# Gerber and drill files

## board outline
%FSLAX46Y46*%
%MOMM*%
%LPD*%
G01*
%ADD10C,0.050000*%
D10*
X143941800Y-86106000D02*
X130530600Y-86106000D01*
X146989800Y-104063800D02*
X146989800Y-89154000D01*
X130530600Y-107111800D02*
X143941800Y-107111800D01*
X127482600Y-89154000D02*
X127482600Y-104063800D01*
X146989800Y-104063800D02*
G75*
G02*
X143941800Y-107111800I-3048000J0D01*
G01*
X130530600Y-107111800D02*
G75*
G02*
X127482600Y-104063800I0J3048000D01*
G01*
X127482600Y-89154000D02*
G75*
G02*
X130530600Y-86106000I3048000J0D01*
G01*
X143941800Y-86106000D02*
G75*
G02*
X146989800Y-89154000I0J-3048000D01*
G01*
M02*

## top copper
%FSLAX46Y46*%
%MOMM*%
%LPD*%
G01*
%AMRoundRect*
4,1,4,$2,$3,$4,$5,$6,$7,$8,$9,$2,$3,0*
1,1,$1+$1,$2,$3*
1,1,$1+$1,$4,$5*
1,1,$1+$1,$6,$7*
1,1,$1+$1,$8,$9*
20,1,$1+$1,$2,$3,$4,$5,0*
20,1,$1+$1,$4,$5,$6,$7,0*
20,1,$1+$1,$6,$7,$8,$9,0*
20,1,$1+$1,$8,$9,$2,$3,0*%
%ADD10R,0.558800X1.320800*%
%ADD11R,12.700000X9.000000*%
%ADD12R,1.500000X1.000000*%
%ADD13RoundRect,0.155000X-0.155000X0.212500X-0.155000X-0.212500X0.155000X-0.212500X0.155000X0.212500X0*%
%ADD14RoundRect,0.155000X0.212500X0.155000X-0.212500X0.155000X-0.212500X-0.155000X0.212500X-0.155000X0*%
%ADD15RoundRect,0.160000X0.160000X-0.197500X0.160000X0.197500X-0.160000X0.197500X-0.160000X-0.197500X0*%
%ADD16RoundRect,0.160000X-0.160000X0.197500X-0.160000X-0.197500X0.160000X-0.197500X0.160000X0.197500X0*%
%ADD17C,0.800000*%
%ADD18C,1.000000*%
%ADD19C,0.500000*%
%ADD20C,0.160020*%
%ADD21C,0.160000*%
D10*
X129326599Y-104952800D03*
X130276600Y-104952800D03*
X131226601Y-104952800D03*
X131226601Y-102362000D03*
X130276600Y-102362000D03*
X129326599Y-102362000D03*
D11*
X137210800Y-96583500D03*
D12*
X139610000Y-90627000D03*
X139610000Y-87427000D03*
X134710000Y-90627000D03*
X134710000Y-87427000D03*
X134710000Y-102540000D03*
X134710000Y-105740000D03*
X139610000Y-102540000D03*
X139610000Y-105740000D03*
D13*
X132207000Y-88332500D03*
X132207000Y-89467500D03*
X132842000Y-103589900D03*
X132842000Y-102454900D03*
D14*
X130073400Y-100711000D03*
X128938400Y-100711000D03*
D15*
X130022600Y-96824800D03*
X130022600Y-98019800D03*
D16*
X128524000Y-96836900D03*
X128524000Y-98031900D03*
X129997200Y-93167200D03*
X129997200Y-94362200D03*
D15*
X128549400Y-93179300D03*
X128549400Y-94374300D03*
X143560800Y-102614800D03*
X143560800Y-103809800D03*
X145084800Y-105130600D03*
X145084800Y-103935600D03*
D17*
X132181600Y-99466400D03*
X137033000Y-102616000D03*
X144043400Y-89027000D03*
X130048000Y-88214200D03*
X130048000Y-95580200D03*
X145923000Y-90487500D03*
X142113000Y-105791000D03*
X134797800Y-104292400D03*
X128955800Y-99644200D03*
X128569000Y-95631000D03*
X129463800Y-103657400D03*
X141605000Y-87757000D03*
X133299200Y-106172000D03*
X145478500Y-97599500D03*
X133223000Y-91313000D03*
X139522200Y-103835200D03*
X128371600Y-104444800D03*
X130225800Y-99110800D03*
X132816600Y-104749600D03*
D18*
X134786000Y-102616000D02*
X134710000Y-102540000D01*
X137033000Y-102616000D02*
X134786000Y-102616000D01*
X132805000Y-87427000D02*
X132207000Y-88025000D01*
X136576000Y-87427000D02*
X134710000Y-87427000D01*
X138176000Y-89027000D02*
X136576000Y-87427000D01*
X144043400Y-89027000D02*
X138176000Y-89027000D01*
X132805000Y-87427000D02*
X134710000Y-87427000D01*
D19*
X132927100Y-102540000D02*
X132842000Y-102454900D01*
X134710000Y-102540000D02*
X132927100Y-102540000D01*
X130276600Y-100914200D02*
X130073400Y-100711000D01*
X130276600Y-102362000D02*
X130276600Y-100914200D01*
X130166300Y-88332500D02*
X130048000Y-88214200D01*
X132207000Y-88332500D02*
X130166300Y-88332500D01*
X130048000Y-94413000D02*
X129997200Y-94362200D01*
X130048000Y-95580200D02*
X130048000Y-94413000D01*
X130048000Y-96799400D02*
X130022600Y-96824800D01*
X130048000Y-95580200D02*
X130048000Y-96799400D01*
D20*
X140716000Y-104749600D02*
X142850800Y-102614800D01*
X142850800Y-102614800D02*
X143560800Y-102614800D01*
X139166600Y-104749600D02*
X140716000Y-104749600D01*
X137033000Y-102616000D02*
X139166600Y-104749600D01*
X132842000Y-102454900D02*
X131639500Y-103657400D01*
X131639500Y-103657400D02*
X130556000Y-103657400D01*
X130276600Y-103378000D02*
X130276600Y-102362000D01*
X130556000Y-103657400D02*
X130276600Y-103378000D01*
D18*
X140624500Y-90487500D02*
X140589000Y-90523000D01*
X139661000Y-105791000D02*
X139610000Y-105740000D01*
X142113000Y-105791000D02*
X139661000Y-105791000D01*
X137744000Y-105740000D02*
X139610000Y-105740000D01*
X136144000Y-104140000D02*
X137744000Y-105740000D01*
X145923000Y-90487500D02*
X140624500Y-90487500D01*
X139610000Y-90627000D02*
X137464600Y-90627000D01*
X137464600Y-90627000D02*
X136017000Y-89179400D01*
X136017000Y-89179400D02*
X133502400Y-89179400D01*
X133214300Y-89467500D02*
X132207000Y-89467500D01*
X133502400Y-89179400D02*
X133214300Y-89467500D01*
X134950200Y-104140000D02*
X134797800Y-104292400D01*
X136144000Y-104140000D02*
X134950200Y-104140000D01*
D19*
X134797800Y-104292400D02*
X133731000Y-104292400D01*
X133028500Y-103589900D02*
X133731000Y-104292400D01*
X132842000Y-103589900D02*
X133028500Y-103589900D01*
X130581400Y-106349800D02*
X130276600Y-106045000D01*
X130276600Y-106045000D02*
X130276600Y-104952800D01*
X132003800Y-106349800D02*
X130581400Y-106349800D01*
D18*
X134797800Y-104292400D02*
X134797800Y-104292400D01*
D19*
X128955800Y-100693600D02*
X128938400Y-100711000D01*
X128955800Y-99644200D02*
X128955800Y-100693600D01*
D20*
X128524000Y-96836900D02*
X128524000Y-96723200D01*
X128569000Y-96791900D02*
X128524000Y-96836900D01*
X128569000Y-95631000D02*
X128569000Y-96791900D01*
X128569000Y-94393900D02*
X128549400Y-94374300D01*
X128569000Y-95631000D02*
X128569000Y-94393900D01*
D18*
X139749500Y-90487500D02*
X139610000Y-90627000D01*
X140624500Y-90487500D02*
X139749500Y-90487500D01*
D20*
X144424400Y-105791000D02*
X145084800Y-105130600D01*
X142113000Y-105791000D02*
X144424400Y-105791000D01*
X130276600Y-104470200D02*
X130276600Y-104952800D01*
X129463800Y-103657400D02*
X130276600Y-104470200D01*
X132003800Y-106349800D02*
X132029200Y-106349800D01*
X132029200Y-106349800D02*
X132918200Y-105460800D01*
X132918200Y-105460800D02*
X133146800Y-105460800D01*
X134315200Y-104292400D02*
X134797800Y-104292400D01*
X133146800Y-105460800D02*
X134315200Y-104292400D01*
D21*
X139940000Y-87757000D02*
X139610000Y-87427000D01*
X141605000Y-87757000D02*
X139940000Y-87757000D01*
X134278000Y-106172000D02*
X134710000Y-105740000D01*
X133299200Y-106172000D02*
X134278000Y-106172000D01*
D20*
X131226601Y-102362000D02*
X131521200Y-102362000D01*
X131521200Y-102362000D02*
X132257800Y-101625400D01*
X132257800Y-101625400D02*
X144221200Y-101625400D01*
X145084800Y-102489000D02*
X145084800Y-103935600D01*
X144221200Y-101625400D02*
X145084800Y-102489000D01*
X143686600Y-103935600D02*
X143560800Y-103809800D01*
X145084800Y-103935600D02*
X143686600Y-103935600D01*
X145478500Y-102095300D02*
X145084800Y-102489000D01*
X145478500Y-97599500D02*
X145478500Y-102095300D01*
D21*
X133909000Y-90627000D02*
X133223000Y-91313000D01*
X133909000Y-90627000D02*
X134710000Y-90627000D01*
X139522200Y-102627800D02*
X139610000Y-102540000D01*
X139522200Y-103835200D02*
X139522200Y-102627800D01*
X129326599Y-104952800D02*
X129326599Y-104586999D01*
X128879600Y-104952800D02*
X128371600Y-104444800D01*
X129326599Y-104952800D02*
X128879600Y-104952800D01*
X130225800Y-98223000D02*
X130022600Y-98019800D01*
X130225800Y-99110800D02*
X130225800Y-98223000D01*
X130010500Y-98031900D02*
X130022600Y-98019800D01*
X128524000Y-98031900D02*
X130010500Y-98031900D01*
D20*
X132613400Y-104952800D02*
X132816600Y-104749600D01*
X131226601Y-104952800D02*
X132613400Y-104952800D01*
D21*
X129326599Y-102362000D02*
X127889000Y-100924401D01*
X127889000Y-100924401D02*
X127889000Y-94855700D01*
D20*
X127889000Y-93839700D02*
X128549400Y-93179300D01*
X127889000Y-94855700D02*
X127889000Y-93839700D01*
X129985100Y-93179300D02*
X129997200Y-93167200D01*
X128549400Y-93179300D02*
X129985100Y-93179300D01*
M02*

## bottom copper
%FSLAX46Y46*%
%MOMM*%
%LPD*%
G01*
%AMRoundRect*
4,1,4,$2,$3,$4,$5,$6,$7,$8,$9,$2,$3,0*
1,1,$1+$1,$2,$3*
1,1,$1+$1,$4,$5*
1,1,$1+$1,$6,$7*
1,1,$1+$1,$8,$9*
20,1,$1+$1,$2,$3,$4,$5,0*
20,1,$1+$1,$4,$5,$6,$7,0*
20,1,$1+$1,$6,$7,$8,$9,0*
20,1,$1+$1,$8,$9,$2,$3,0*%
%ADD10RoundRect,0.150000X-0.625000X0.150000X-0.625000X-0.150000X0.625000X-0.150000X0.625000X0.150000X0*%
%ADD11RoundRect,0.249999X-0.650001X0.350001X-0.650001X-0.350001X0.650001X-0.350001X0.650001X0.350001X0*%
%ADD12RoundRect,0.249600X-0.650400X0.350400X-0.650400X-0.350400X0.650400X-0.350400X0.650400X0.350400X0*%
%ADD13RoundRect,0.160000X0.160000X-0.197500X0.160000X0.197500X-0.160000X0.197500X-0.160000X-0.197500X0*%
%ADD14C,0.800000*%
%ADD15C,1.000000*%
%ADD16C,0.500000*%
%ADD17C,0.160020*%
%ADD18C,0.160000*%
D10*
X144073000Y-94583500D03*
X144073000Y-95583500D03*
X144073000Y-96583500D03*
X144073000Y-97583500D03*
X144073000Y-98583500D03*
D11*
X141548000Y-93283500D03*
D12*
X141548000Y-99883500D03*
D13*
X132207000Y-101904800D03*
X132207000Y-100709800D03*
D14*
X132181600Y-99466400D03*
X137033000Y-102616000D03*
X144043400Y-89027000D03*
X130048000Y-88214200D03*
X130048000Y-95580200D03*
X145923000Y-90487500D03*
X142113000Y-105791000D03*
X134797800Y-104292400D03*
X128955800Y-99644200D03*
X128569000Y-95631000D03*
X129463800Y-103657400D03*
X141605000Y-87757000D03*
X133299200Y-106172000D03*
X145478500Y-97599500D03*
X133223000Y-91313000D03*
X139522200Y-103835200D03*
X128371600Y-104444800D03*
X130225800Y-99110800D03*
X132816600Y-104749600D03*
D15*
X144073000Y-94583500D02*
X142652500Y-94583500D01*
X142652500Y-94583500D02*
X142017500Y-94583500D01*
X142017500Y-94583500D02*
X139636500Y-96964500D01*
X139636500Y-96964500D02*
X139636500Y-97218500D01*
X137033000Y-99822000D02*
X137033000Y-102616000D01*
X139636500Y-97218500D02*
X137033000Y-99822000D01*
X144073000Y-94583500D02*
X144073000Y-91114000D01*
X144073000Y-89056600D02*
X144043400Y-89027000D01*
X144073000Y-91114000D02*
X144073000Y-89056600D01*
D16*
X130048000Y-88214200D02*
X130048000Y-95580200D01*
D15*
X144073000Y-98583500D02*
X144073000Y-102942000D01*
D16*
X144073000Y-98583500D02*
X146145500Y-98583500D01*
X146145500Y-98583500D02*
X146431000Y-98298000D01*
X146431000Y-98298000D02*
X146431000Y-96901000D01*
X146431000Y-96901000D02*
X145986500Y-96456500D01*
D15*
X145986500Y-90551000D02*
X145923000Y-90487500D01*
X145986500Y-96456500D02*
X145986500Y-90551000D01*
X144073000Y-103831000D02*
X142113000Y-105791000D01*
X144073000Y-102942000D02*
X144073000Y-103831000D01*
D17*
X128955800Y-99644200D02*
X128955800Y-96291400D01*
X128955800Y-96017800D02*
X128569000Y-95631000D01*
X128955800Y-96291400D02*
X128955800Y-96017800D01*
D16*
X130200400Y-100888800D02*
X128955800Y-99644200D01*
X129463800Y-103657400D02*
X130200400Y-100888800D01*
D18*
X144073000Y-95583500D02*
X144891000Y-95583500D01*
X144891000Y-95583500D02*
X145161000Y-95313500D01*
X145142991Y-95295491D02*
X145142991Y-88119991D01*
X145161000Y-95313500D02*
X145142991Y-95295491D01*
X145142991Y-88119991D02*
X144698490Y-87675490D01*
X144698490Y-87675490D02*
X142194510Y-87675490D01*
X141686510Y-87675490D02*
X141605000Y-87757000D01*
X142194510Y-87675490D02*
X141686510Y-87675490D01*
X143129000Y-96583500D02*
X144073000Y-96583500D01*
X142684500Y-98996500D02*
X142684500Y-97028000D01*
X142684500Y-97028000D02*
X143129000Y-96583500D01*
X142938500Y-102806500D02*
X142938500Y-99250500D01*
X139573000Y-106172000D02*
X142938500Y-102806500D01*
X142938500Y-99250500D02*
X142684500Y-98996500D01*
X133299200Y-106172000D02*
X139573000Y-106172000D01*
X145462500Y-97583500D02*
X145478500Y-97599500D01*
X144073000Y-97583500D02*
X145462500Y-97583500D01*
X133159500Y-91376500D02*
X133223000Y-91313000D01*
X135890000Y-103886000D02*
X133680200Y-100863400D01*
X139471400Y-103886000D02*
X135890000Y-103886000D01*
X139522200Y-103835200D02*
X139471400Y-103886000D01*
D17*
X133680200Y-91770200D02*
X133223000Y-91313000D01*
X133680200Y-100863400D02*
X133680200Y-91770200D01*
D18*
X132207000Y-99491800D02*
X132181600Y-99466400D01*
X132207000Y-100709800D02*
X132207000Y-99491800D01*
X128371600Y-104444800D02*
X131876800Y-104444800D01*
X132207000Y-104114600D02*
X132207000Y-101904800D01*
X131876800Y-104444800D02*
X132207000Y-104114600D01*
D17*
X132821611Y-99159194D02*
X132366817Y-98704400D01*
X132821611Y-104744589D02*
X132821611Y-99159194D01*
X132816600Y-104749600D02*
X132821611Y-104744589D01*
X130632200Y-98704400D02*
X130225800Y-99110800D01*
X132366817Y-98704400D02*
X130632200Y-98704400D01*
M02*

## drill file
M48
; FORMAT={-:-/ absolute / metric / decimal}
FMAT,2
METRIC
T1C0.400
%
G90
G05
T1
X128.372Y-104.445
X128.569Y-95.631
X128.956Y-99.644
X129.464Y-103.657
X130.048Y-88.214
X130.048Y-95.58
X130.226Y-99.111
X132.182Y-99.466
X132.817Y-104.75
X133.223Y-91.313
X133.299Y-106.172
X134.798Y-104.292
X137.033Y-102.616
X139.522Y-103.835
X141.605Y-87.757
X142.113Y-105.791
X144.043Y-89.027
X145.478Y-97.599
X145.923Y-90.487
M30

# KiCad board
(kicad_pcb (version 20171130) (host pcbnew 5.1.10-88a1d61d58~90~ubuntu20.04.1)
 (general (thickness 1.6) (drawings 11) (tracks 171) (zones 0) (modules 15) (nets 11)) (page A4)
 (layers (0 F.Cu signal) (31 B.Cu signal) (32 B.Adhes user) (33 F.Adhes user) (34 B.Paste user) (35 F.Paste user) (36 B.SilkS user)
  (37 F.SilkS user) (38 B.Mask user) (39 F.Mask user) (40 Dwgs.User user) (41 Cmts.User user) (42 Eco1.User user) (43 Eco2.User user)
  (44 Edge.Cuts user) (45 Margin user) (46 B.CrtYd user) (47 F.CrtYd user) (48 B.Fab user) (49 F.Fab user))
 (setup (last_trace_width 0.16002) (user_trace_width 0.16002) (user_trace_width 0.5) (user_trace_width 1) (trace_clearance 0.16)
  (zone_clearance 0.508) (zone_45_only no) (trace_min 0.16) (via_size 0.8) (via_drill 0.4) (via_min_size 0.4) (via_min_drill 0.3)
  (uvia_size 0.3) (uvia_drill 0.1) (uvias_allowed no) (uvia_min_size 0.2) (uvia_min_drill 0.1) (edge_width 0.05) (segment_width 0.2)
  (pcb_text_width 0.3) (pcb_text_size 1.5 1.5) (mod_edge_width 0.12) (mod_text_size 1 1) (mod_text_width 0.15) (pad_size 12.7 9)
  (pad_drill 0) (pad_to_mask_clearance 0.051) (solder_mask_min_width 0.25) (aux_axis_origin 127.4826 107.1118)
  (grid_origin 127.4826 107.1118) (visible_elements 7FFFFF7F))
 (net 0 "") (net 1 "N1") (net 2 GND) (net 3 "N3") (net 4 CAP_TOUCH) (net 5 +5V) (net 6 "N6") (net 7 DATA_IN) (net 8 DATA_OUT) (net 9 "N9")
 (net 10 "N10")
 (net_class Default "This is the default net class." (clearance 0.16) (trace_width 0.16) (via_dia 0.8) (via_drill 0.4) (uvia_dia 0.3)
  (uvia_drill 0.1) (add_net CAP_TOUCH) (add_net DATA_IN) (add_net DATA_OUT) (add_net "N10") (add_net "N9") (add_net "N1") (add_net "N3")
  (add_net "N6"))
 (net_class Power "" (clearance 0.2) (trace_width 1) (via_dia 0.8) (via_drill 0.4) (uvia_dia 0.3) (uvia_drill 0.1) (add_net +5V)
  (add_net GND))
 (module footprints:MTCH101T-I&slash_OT (layer F.Cu) (at 130.2766 103.6574 90)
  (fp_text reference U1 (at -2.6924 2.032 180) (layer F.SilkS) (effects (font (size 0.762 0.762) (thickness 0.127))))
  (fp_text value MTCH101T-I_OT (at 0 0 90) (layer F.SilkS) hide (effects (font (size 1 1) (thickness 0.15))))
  (pad 1 smd rect (at -1.2954 -0.950001 90) (size 1.3208 0.5588) (layers F.Cu F.Paste F.Mask) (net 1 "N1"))
  (pad 2 smd rect (at -1.2954 0 90) (size 1.3208 0.5588) (layers F.Cu F.Paste F.Mask) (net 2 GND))
  (pad 3 smd rect (at -1.2954 0.950001 90) (size 1.3208 0.5588) (layers F.Cu F.Paste F.Mask) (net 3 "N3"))
  (pad 4 smd rect (at 1.2954 0.950001 90) (size 1.3208 0.5588) (layers F.Cu F.Paste F.Mask) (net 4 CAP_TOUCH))
  (pad 5 smd rect (at 1.2954 0 90) (size 1.3208 0.5588) (layers F.Cu F.Paste F.Mask) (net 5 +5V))
  (pad 6 smd rect (at 1.2954 -0.950001 90) (size 1.3208 0.5588) (layers F.Cu F.Paste F.Mask) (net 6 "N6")))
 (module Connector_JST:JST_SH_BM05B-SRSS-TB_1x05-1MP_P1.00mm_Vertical (layer B.Cu) (at 142.748 96.5835 270)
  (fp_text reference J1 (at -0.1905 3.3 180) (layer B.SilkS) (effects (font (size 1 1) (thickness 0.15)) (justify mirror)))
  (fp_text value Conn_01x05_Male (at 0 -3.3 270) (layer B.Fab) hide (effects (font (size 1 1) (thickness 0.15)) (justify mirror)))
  (pad 1 smd roundrect (at -2 -1.325 270) (size 0.6 1.55) (layers B.Cu B.Mask) (roundrect_rratio 0.25) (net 5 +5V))
  (pad 2 smd roundrect (at -1 -1.325 270) (size 0.6 1.55) (layers B.Cu B.Mask) (roundrect_rratio 0.25) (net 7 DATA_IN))
  (pad 3 smd roundrect (at 0 -1.325 270) (size 0.6 1.55) (layers B.Cu B.Mask) (roundrect_rratio 0.25) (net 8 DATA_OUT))
  (pad 4 smd roundrect (at 1 -1.325 270) (size 0.6 1.55) (layers B.Cu B.Mask) (roundrect_rratio 0.25) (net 4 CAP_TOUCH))
  (pad 5 smd roundrect (at 2 -1.325 270) (size 0.6 1.55) (layers B.Cu B.Mask) (roundrect_rratio 0.25) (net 2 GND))
  (pad MP smd roundrect (at -3.3 1.2 270) (size 1.2 1.8) (layers B.Cu B.Paste B.Mask) (roundrect_rratio 0.2083325))
  (pad MP smd roundrect (at 3.3 1.2 270) (size 1.2 1.8) (layers B.Cu B.Mask) (roundrect_rratio 0.208)))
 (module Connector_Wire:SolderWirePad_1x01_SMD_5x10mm (layer F.Cu) (at 136.0805 96.647)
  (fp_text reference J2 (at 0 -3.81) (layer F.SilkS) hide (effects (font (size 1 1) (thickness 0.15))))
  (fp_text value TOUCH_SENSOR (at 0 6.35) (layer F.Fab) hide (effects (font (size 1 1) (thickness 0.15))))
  (pad 1 smd rect (at 1.1303 -0.0635) (size 12.7 9) (layers F.Cu F.Mask) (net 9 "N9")))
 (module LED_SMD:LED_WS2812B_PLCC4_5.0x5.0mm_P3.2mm (layer F.Cu) (at 137.16 89.027)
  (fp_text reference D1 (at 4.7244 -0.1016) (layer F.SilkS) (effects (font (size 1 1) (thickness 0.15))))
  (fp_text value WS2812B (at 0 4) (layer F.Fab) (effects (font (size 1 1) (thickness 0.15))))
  (pad 3 smd rect (at 2.45 1.6) (size 1.5 1) (layers F.Cu F.Paste F.Mask) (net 2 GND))
  (pad 4 smd rect (at 2.45 -1.6) (size 1.5 1) (layers F.Cu F.Paste F.Mask) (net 7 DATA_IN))
  (pad 2 smd rect (at -2.45 1.6) (size 1.5 1) (layers F.Cu F.Paste F.Mask) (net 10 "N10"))
  (pad 1 smd rect (at -2.45 -1.6) (size 1.5 1) (layers F.Cu F.Paste F.Mask) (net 5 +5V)))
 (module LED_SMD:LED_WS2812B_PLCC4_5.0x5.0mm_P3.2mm (layer F.Cu) (at 137.16 104.14)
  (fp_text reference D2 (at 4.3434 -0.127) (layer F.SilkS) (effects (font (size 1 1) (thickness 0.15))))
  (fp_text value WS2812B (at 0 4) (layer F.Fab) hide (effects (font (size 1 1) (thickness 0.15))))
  (pad 1 smd rect (at -2.45 -1.6) (size 1.5 1) (layers F.Cu F.Paste F.Mask) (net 5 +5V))
  (pad 2 smd rect (at -2.45 1.6) (size 1.5 1) (layers F.Cu F.Paste F.Mask) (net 8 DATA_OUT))
  (pad 4 smd rect (at 2.45 -1.6) (size 1.5 1) (layers F.Cu F.Paste F.Mask) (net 10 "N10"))
  (pad 3 smd rect (at 2.45 1.6) (size 1.5 1) (layers F.Cu F.Paste F.Mask) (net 2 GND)))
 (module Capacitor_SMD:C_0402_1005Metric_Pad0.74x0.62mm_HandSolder (layer F.Cu) (at 132.207 88.9 270)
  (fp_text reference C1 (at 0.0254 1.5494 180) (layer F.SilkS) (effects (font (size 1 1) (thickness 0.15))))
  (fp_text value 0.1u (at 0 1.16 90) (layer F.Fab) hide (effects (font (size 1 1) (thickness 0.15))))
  (pad 1 smd roundrect (at -0.5675 0 270) (size 0.735 0.62) (layers F.Cu F.Paste F.Mask) (roundrect_rratio 0.25) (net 5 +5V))
  (pad 2 smd roundrect (at 0.5675 0 270) (size 0.735 0.62) (layers F.Cu F.Paste F.Mask) (roundrect_rratio 0.25) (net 2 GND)))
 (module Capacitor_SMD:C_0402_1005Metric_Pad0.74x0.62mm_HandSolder (layer F.Cu) (at 132.842 103.0224 270)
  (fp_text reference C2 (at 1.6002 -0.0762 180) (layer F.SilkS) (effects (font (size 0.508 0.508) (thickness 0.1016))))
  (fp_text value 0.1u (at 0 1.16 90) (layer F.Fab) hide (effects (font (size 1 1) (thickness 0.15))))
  (pad 2 smd roundrect (at 0.5675 0 270) (size 0.735 0.62) (layers F.Cu F.Paste F.Mask) (roundrect_rratio 0.25) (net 2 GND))
  (pad 1 smd roundrect (at -0.5675 0 270) (size 0.735 0.62) (layers F.Cu F.Paste F.Mask) (roundrect_rratio 0.25) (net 5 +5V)))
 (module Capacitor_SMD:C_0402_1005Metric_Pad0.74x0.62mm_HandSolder (layer F.Cu) (at 129.5059 100.711 180)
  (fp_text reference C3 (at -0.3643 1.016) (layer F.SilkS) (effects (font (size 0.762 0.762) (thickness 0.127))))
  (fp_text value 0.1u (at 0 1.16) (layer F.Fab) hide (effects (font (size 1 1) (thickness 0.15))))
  (pad 1 smd roundrect (at -0.5675 0 180) (size 0.735 0.62) (layers F.Cu F.Paste F.Mask) (roundrect_rratio 0.25) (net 5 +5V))
  (pad 2 smd roundrect (at 0.5675 0 180) (size 0.735 0.62) (layers F.Cu F.Paste F.Mask) (roundrect_rratio 0.25) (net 2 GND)))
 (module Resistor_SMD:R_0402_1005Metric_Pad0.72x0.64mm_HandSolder (layer B.Cu) (at 132.207 101.3073 90)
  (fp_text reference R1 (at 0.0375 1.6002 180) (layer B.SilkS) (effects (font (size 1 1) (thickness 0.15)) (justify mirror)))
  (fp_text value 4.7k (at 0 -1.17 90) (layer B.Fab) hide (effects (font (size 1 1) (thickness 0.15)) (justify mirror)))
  (pad 1 smd roundrect (at -0.5975 0 90) (size 0.715 0.64) (layers B.Cu B.Paste B.Mask) (roundrect_rratio 0.25) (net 1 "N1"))
  (pad 2 smd roundrect (at 0.5975 0 90) (size 0.715 0.64) (layers B.Cu B.Paste B.Mask) (roundrect_rratio 0.25) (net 9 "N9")))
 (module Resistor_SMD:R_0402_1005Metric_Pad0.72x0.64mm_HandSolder (layer F.Cu) (at 130.0226 97.4223 90)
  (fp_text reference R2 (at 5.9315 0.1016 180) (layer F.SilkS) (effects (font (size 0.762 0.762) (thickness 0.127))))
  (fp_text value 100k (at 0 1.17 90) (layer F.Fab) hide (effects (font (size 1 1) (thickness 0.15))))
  (pad 2 smd roundrect (at 0.5975 0 90) (size 0.715 0.64) (layers F.Cu F.Paste F.Mask) (roundrect_rratio 0.25) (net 5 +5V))
  (pad 1 smd roundrect (at -0.5975 0 90) (size 0.715 0.64) (layers F.Cu F.Paste F.Mask) (roundrect_rratio 0.25) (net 3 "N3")))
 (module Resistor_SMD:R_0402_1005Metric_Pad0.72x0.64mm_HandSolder (layer F.Cu) (at 128.524 97.4344 270)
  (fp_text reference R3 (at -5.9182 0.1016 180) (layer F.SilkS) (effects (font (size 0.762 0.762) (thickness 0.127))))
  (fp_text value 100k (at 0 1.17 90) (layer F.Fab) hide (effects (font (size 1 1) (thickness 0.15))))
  (pad 1 smd roundrect (at -0.5975 0 270) (size 0.715 0.64) (layers F.Cu F.Paste F.Mask) (roundrect_rratio 0.25) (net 2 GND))
  (pad 2 smd roundrect (at 0.5975 0 270) (size 0.715 0.64) (layers F.Cu F.Paste F.Mask) (roundrect_rratio 0.25) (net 3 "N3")))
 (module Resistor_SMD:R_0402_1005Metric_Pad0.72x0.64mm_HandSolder (layer F.Cu) (at 129.9972 93.7647 270)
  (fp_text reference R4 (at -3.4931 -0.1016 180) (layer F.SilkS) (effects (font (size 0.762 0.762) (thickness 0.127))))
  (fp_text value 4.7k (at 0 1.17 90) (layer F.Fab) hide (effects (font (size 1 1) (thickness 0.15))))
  (pad 1 smd roundrect (at -0.5975 0 270) (size 0.715 0.64) (layers F.Cu F.Paste F.Mask) (roundrect_rratio 0.25) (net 6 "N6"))
  (pad 2 smd roundrect (at 0.5975 0 270) (size 0.715 0.64) (layers F.Cu F.Paste F.Mask) (roundrect_rratio 0.25) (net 5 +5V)))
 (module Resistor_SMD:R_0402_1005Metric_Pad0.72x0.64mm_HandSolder (layer F.Cu) (at 128.5494 93.7768 90)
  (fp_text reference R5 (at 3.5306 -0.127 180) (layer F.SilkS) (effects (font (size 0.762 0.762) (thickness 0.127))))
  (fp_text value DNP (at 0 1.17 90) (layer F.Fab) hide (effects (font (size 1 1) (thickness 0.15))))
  (pad 2 smd roundrect (at 0.5975 0 90) (size 0.715 0.64) (layers F.Cu F.Paste F.Mask) (roundrect_rratio 0.25) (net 6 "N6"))
  (pad 1 smd roundrect (at -0.5975 0 90) (size 0.715 0.64) (layers F.Cu F.Paste F.Mask) (roundrect_rratio 0.25) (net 2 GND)))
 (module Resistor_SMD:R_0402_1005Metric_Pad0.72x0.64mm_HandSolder (layer F.Cu) (at 143.5608 103.2123 90)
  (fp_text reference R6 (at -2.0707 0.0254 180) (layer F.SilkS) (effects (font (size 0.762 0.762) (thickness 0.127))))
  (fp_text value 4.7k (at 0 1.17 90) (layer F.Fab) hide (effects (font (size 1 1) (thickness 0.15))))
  (pad 2 smd roundrect (at 0.5975 0 90) (size 0.715 0.64) (layers F.Cu F.Paste F.Mask) (roundrect_rratio 0.25) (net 5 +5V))
  (pad 1 smd roundrect (at -0.5975 0 90) (size 0.715 0.64) (layers F.Cu F.Paste F.Mask) (roundrect_rratio 0.25) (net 4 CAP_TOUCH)))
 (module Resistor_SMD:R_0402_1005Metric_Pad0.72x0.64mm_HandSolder (layer F.Cu) (at 145.0848 104.5331 90)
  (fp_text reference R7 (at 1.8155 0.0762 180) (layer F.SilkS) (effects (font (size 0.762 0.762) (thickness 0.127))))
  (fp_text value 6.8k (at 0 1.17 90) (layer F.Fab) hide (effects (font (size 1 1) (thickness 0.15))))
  (pad 1 smd roundrect (at -0.5975 0 90) (size 0.715 0.64) (layers F.Cu F.Paste F.Mask) (roundrect_rratio 0.25) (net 2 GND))
  (pad 2 smd roundrect (at 0.5975 0 90) (size 0.715 0.64) (layers F.Cu F.Paste F.Mask) (roundrect_rratio 0.25) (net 4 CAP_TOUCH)))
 (gr_line (start 143.9418 86.106) (end 130.5306 86.106) (layer Edge.Cuts) (width 0.05))
 (gr_line (start 146.9898 104.0638) (end 146.9898 89.154) (layer Edge.Cuts) (width 0.05))
 (gr_line (start 130.5306 107.1118) (end 143.9418 107.1118) (layer Edge.Cuts) (width 0.05))
 (gr_line (start 127.4826 89.154) (end 127.4826 104.0638) (layer Edge.Cuts) (width 0.05))
 (gr_arc (start 143.9418 104.0638) (end 143.9418 107.1118) (angle -90) (layer Edge.Cuts) (width 0.05))
 (gr_arc (start 130.5306 104.0638) (end 127.4826 104.0638) (angle -90) (layer Edge.Cuts) (width 0.05))
 (gr_arc (start 130.5306 89.154) (end 130.5306 86.106) (angle -90) (layer Edge.Cuts) (width 0.05))
 (gr_arc (start 143.9418 89.154) (end 146.9898 89.154) (angle -90) (layer Edge.Cuts) (width 0.05))
 (via (at 132.1816 99.4664) (size 0.8) (drill 0.4) (layers F.Cu B.Cu) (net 9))
 (segment (start 144.073 94.5835) (end 142.6525 94.5835) (width 1) (layer B.Cu) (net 5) (status 10))
 (segment (start 142.6525 94.5835) (end 142.0175 94.5835) (width 1) (layer B.Cu) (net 5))
 (segment (start 142.0175 94.5835) (end 139.6365 96.9645) (width 1) (layer B.Cu) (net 5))
 (segment (start 139.6365 96.9645) (end 139.6365 97.2185) (width 1) (layer B.Cu) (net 5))
 (via (at 137.033 102.616) (size 0.8) (drill 0.4) (layers F.Cu B.Cu) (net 5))
 (segment (start 137.033 99.822) (end 137.033 102.616) (width 1) (layer B.Cu) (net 5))
 (segment (start 139.6365 97.2185) (end 137.033 99.822) (width 1) (layer B.Cu) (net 5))
 (segment (start 134.786 102.616) (end 134.71 102.54) (width 1) (layer F.Cu) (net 5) (status 30))
 (segment (start 137.033 102.616) (end 134.786 102.616) (width 1) (layer F.Cu) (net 5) (status 20))
 (segment (start 144.073 94.5835) (end 144.073 91.114) (width 1) (layer B.Cu) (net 5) (status 10))
 (segment (start 132.805 87.427) (end 132.207 88.025) (width 1) (layer F.Cu) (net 5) (status 20))
 (via (at 144.0434 89.027) (size 0.8) (drill 0.4) (layers F.Cu B.Cu) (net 5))
 (segment (start 144.073 89.0566) (end 144.0434 89.027) (width 1) (layer B.Cu) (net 5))
 (segment (start 144.073 91.114) (end 144.073 89.0566) (width 1) (layer B.Cu) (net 5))
 (segment (start 136.576 87.427) (end 134.71 87.427) (width 1) (layer F.Cu) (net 5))
 (segment (start 138.176 89.027) (end 136.576 87.427) (width 1) (layer F.Cu) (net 5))
 (segment (start 144.0434 89.027) (end 138.176 89.027) (width 1) (layer F.Cu) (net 5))
 (segment (start 132.805 87.427) (end 134.71 87.427) (width 1) (layer F.Cu) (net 5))
 (segment (start 132.9271 102.54) (end 132.842 102.4549) (width 0.5) (layer F.Cu) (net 5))
 (segment (start 134.71 102.54) (end 132.9271 102.54) (width 0.5) (layer F.Cu) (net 5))
 (segment (start 130.2766 100.9142) (end 130.0734 100.711) (width 0.5) (layer F.Cu) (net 5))
 (segment (start 130.2766 102.362) (end 130.2766 100.9142) (width 0.5) (layer F.Cu) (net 5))
 (via (at 130.048 88.2142) (size 0.8) (drill 0.4) (layers F.Cu B.Cu) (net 5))
 (segment (start 130.1663 88.3325) (end 130.048 88.2142) (width 0.5) (layer F.Cu) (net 5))
 (segment (start 132.207 88.3325) (end 130.1663 88.3325) (width 0.5) (layer F.Cu) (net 5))
 (via (at 130.048 95.5802) (size 0.8) (drill 0.4) (layers F.Cu B.Cu) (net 5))
 (segment (start 130.048 88.2142) (end 130.048 95.5802) (width 0.5) (layer B.Cu) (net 5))
 (segment (start 130.048 94.413) (end 129.9972 94.3622) (width 0.5) (layer F.Cu) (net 5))
 (segment (start 130.048 95.5802) (end 130.048 94.413) (width 0.5) (layer F.Cu) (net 5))
 (segment (start 130.048 96.7994) (end 130.0226 96.8248) (width 0.5) (layer F.Cu) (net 5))
 (segment (start 130.048 95.5802) (end 130.048 96.7994) (width 0.5) (layer F.Cu) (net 5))
 (segment (start 140.716 104.7496) (end 142.8508 102.6148) (width 0.16002) (layer F.Cu) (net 5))
 (segment (start 142.8508 102.6148) (end 143.5608 102.6148) (width 0.16002) (layer F.Cu) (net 5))
 (segment (start 139.1666 104.7496) (end 140.716 104.7496) (width 0.16002) (layer F.Cu) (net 5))
 (segment (start 137.033 102.616) (end 139.1666 104.7496) (width 0.16002) (layer F.Cu) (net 5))
 (segment (start 132.842 102.4549) (end 131.6395 103.6574) (width 0.16002) (layer F.Cu) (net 5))
 (segment (start 131.6395 103.6574) (end 130.556 103.6574) (width 0.16002) (layer F.Cu) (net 5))
 (segment (start 130.2766 103.378) (end 130.2766 102.362) (width 0.16002) (layer F.Cu) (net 5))
 (segment (start 130.556 103.6574) (end 130.2766 103.378) (width 0.16002) (layer F.Cu) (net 5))
 (segment (start 144.073 98.5835) (end 144.073 102.942) (width 1) (layer B.Cu) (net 2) (status 10))
 (segment (start 144.073 98.5835) (end 146.1455 98.5835) (width 0.5) (layer B.Cu) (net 2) (status 10))
 (segment (start 146.1455 98.5835) (end 146.431 98.298) (width 0.5) (layer B.Cu) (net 2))
 (segment (start 146.431 98.298) (end 146.431 96.901) (width 0.5) (layer B.Cu) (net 2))
 (segment (start 146.431 96.901) (end 145.9865 96.4565) (width 0.5) (layer B.Cu) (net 2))
 (via (at 145.923 90.4875) (size 0.8) (drill 0.4) (layers F.Cu B.Cu) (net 2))
 (segment (start 140.6245 90.4875) (end 140.589 90.523) (width 1) (layer F.Cu) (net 2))
 (segment (start 145.9865 90.551) (end 145.923 90.4875) (width 1) (layer B.Cu) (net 2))
 (segment (start 145.9865 96.4565) (end 145.9865 90.551) (width 1) (layer B.Cu) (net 2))
 (via (at 142.113 105.791) (size 0.8) (drill 0.4) (layers F.Cu B.Cu) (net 2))
 (segment (start 144.073 103.831) (end 142.113 105.791) (width 1) (layer B.Cu) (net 2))
 (segment (start 144.073 102.942) (end 144.073 103.831) (width 1) (layer B.Cu) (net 2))
 (segment (start 139.661 105.791) (end 139.61 105.74) (width 1) (layer F.Cu) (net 2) (status 30))
 (segment (start 142.113 105.791) (end 139.661 105.791) (width 1) (layer F.Cu) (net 2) (status 20))
 (segment (start 137.744 105.74) (end 139.61 105.74) (width 1) (layer F.Cu) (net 2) (status 20))
 (segment (start 136.144 104.14) (end 137.744 105.74) (width 1) (layer F.Cu) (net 2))
 (segment (start 145.923 90.4875) (end 140.6245 90.4875) (width 1) (layer F.Cu) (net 2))
 (segment (start 139.61 90.627) (end 137.4646 90.627) (width 1) (layer F.Cu) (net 2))
 (segment (start 137.4646 90.627) (end 136.017 89.1794) (width 1) (layer F.Cu) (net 2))
 (segment (start 136.017 89.1794) (end 133.5024 89.1794) (width 1) (layer F.Cu) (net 2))
 (segment (start 133.2143 89.4675) (end 132.207 89.4675) (width 1) (layer F.Cu) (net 2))
 (segment (start 133.5024 89.1794) (end 133.2143 89.4675) (width 1) (layer F.Cu) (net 2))
 (segment (start 134.9502 104.14) (end 134.7978 104.2924) (width 1) (layer F.Cu) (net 2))
 (segment (start 136.144 104.14) (end 134.9502 104.14) (width 1) (layer F.Cu) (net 2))
 (segment (start 134.7978 104.2924) (end 133.731 104.2924) (width 0.5) (layer F.Cu) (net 2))
 (segment (start 133.0285 103.5899) (end 133.731 104.2924) (width 0.5) (layer F.Cu) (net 2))
 (segment (start 132.842 103.5899) (end 133.0285 103.5899) (width 0.5) (layer F.Cu) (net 2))
 (segment (start 130.5814 106.3498) (end 130.2766 106.045) (width 0.5) (layer F.Cu) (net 2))
 (segment (start 130.2766 106.045) (end 130.2766 104.9528) (width 0.5) (layer F.Cu) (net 2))
 (segment (start 132.0038 106.3498) (end 130.5814 106.3498) (width 0.5) (layer F.Cu) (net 2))
 (segment (start 134.7978 104.2924) (end 134.7978 104.2924) (width 1) (layer F.Cu) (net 2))
 (via (at 134.7978 104.2924) (size 0.8) (drill 0.4) (layers F.Cu B.Cu) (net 2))
 (via (at 128.9558 99.6442) (size 0.8) (drill 0.4) (layers F.Cu B.Cu) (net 2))
 (segment (start 128.9558 100.6936) (end 128.9384 100.711) (width 0.5) (layer F.Cu) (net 2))
 (segment (start 128.9558 99.6442) (end 128.9558 100.6936) (width 0.5) (layer F.Cu) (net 2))
 (segment (start 128.9558 99.6442) (end 128.9558 96.2914) (width 0.16002) (layer B.Cu) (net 2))
 (segment (start 128.524 96.8369) (end 128.524 96.7232) (width 0.16002) (layer F.Cu) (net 2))
 (via (at 128.569 95.631) (size 0.8) (drill 0.4) (layers F.Cu B.Cu) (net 2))
 (segment (start 128.9558 96.0178) (end 128.569 95.631) (width 0.16002) (layer B.Cu) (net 2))
 (segment (start 128.9558 96.2914) (end 128.9558 96.0178) (width 0.16002) (layer B.Cu) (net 2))
 (segment (start 128.569 96.7919) (end 128.524 96.8369) (width 0.16002) (layer F.Cu) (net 2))
 (segment (start 128.569 95.631) (end 128.569 96.7919) (width 0.16002) (layer F.Cu) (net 2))
 (segment (start 128.569 94.3939) (end 128.5494 94.3743) (width 0.16002) (layer F.Cu) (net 2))
 (segment (start 128.569 95.631) (end 128.569 94.3939) (width 0.16002) (layer F.Cu) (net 2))
 (segment (start 139.7495 90.4875) (end 139.61 90.627) (width 1) (layer F.Cu) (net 2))
 (segment (start 140.6245 90.4875) (end 139.7495 90.4875) (width 1) (layer F.Cu) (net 2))
 (segment (start 144.4244 105.791) (end 145.0848 105.1306) (width 0.16002) (layer F.Cu) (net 2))
 (segment (start 142.113 105.791) (end 144.4244 105.791) (width 0.16002) (layer F.Cu) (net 2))
 (segment (start 130.2004 100.8888) (end 128.9558 99.6442) (width 0.5) (layer B.Cu) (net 2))
 (segment (start 129.4638 103.6574) (end 130.2004 100.8888) (width 0.5) (layer B.Cu) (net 2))
 (via (at 129.4638 103.6574) (size 0.8) (drill 0.4) (layers F.Cu B.Cu) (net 2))
 (segment (start 130.2766 104.4702) (end 130.2766 104.9528) (width 0.16002) (layer F.Cu) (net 2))
 (segment (start 129.4638 103.6574) (end 130.2766 104.4702) (width 0.16002) (layer F.Cu) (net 2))
 (segment (start 132.0038 106.3498) (end 132.0292 106.3498) (width 0.16002) (layer F.Cu) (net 2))
 (segment (start 132.0292 106.3498) (end 132.9182 105.4608) (width 0.16002) (layer F.Cu) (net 2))
 (segment (start 132.9182 105.4608) (end 133.1468 105.4608) (width 0.16002) (layer F.Cu) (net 2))
 (segment (start 134.3152 104.2924) (end 134.7978 104.2924) (width 0.16002) (layer F.Cu) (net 2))
 (segment (start 133.1468 105.4608) (end 134.3152 104.2924) (width 0.16002) (layer F.Cu) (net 2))
 (segment (start 144.073 95.5835) (end 144.891 95.5835) (width 0.16) (layer B.Cu) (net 7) (status 10))
 (segment (start 144.891 95.5835) (end 145.161 95.3135) (width 0.16) (layer B.Cu) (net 7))
 (segment (start 145.142991 95.295491) (end 145.142991 88.119991) (width 0.16) (layer B.Cu) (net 7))
 (segment (start 145.161 95.3135) (end 145.142991 95.295491) (width 0.16) (layer B.Cu) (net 7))
 (segment (start 145.142991 88.119991) (end 144.69849 87.67549) (width 0.16) (layer B.Cu) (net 7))
 (segment (start 144.69849 87.67549) (end 142.19451 87.67549) (width 0.16) (layer B.Cu) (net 7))
 (via (at 141.605 87.757) (size 0.8) (drill 0.4) (layers F.Cu B.Cu) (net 7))
 (segment (start 141.68651 87.67549) (end 141.605 87.757) (width 0.16) (layer B.Cu) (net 7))
 (segment (start 142.19451 87.67549) (end 141.68651 87.67549) (width 0.16) (layer B.Cu) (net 7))
 (segment (start 139.94 87.757) (end 139.61 87.427) (width 0.16) (layer F.Cu) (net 7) (status 30))
 (segment (start 141.605 87.757) (end 139.94 87.757) (width 0.16) (layer F.Cu) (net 7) (status 20))
 (segment (start 134.278 106.172) (end 134.71 105.74) (width 0.16) (layer F.Cu) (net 8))
 (segment (start 133.2992 106.172) (end 134.278 106.172) (width 0.16) (layer F.Cu) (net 8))
 (segment (start 143.129 96.5835) (end 144.073 96.5835) (width 0.16) (layer B.Cu) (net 8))
 (segment (start 142.6845 98.9965) (end 142.6845 97.028) (width 0.16) (layer B.Cu) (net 8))
 (segment (start 142.6845 97.028) (end 143.129 96.5835) (width 0.16) (layer B.Cu) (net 8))
 (segment (start 142.9385 102.8065) (end 142.9385 99.2505) (width 0.16) (layer B.Cu) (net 8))
 (segment (start 139.573 106.172) (end 142.9385 102.8065) (width 0.16) (layer B.Cu) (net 8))
 (segment (start 142.9385 99.2505) (end 142.6845 98.9965) (width 0.16) (layer B.Cu) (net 8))
 (segment (start 133.2992 106.172) (end 139.573 106.172) (width 0.16) (layer B.Cu) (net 8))
 (via (at 133.2992 106.172) (size 0.8) (drill 0.4) (layers F.Cu B.Cu) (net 8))
 (via (at 145.4785 97.5995) (size 0.8) (drill 0.4) (layers F.Cu B.Cu) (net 4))
 (segment (start 145.4625 97.5835) (end 145.4785 97.5995) (width 0.16) (layer B.Cu) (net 4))
 (segment (start 144.073 97.5835) (end 145.4625 97.5835) (width 0.16) (layer B.Cu) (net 4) (status 10))
 (segment (start 131.226601 102.362) (end 131.5212 102.362) (width 0.16002) (layer F.Cu) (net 4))
 (segment (start 131.5212 102.362) (end 132.2578 101.6254) (width 0.16002) (layer F.Cu) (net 4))
 (segment (start 132.2578 101.6254) (end 144.2212 101.6254) (width 0.16002) (layer F.Cu) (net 4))
 (segment (start 145.0848 102.489) (end 145.0848 103.9356) (width 0.16002) (layer F.Cu) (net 4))
 (segment (start 144.2212 101.6254) (end 145.0848 102.489) (width 0.16002) (layer F.Cu) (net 4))
 (segment (start 143.6866 103.9356) (end 143.5608 103.8098) (width 0.16002) (layer F.Cu) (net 4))
 (segment (start 145.0848 103.9356) (end 143.6866 103.9356) (width 0.16002) (layer F.Cu) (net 4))
 (segment (start 145.4785 102.0953) (end 145.0848 102.489) (width 0.16002) (layer F.Cu) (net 4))
 (segment (start 145.4785 97.5995) (end 145.4785 102.0953) (width 0.16002) (layer F.Cu) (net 4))
 (via (at 133.223 91.313) (size 0.8) (drill 0.4) (layers F.Cu B.Cu) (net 10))
 (segment (start 133.909 90.627) (end 133.223 91.313) (width 0.16) (layer F.Cu) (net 10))
 (via (at 139.5222 103.8352) (size 0.8) (drill 0.4) (layers F.Cu B.Cu) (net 10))
 (segment (start 133.909 90.627) (end 134.71 90.627) (width 0.16) (layer F.Cu) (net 10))
 (segment (start 139.5222 102.6278) (end 139.61 102.54) (width 0.16) (layer F.Cu) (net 10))
 (segment (start 139.5222 103.8352) (end 139.5222 102.6278) (width 0.16) (layer F.Cu) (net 10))
 (segment (start 133.1595 91.3765) (end 133.223 91.313) (width 0.16) (layer B.Cu) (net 10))
 (segment (start 135.89 103.886) (end 133.6802 100.8634) (width 0.16) (layer B.Cu) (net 10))
 (segment (start 139.4714 103.886) (end 135.89 103.886) (width 0.16) (layer B.Cu) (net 10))
 (segment (start 139.5222 103.8352) (end 139.4714 103.886) (width 0.16) (layer B.Cu) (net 10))
 (segment (start 133.6802 91.7702) (end 133.223 91.313) (width 0.16002) (layer B.Cu) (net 10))
 (segment (start 133.6802 100.8634) (end 133.6802 91.7702) (width 0.16002) (layer B.Cu) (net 10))
 (segment (start 132.207 99.4918) (end 132.1816 99.4664) (width 0.16) (layer B.Cu) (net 9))
 (segment (start 132.207 100.7098) (end 132.207 99.4918) (width 0.16) (layer B.Cu) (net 9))
 (segment (start 129.326599 104.9528) (end 129.326599 104.586999) (width 0.16) (layer F.Cu) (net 1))
 (via (at 128.3716 104.4448) (size 0.8) (drill 0.4) (layers F.Cu B.Cu) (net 1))
 (segment (start 128.8796 104.9528) (end 128.3716 104.4448) (width 0.16) (layer F.Cu) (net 1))
 (segment (start 129.326599 104.9528) (end 128.8796 104.9528) (width 0.16) (layer F.Cu) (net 1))
 (segment (start 128.3716 104.4448) (end 131.8768 104.4448) (width 0.16) (layer B.Cu) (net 1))
 (segment (start 132.207 104.1146) (end 132.207 101.9048) (width 0.16) (layer B.Cu) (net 1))
 (segment (start 131.8768 104.4448) (end 132.207 104.1146) (width 0.16) (layer B.Cu) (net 1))
 (via (at 130.2258 99.1108) (size 0.8) (drill 0.4) (layers F.Cu B.Cu) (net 3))
 (segment (start 130.2258 98.223) (end 130.0226 98.0198) (width 0.16) (layer F.Cu) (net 3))
 (segment (start 130.2258 99.1108) (end 130.2258 98.223) (width 0.16) (layer F.Cu) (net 3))
 (segment (start 130.0105 98.0319) (end 130.0226 98.0198) (width 0.16) (layer F.Cu) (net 3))
 (segment (start 128.524 98.0319) (end 130.0105 98.0319) (width 0.16) (layer F.Cu) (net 3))
 (via (at 132.8166 104.7496) (size 0.8) (drill 0.4) (layers F.Cu B.Cu) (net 3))
 (segment (start 132.6134 104.9528) (end 132.8166 104.7496) (width 0.16002) (layer F.Cu) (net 3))
 (segment (start 131.226601 104.9528) (end 132.6134 104.9528) (width 0.16002) (layer F.Cu) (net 3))
 (segment (start 132.821611 99.159194) (end 132.366817 98.7044) (width 0.16002) (layer B.Cu) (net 3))
 (segment (start 132.821611 104.744589) (end 132.821611 99.159194) (width 0.16002) (layer B.Cu) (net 3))
 (segment (start 132.8166 104.7496) (end 132.821611 104.744589) (width 0.16002) (layer B.Cu) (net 3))
 (segment (start 130.6322 98.7044) (end 130.2258 99.1108) (width 0.16002) (layer B.Cu) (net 3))
 (segment (start 132.366817 98.7044) (end 130.6322 98.7044) (width 0.16002) (layer B.Cu) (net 3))
 (segment (start 129.326599 102.362) (end 127.889 100.924401) (width 0.16) (layer F.Cu) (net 6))
 (segment (start 127.889 100.924401) (end 127.889 94.8557) (width 0.16) (layer F.Cu) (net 6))
 (segment (start 127.889 93.8397) (end 128.5494 93.1793) (width 0.16002) (layer F.Cu) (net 6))
 (segment (start 127.889 94.8557) (end 127.889 93.8397) (width 0.16002) (layer F.Cu) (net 6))
 (segment (start 129.9851 93.1793) (end 129.9972 93.1672) (width 0.16002) (layer F.Cu) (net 6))
 (segment (start 128.5494 93.1793) (end 129.9851 93.1793) (width 0.16002) (layer F.Cu) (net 6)))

